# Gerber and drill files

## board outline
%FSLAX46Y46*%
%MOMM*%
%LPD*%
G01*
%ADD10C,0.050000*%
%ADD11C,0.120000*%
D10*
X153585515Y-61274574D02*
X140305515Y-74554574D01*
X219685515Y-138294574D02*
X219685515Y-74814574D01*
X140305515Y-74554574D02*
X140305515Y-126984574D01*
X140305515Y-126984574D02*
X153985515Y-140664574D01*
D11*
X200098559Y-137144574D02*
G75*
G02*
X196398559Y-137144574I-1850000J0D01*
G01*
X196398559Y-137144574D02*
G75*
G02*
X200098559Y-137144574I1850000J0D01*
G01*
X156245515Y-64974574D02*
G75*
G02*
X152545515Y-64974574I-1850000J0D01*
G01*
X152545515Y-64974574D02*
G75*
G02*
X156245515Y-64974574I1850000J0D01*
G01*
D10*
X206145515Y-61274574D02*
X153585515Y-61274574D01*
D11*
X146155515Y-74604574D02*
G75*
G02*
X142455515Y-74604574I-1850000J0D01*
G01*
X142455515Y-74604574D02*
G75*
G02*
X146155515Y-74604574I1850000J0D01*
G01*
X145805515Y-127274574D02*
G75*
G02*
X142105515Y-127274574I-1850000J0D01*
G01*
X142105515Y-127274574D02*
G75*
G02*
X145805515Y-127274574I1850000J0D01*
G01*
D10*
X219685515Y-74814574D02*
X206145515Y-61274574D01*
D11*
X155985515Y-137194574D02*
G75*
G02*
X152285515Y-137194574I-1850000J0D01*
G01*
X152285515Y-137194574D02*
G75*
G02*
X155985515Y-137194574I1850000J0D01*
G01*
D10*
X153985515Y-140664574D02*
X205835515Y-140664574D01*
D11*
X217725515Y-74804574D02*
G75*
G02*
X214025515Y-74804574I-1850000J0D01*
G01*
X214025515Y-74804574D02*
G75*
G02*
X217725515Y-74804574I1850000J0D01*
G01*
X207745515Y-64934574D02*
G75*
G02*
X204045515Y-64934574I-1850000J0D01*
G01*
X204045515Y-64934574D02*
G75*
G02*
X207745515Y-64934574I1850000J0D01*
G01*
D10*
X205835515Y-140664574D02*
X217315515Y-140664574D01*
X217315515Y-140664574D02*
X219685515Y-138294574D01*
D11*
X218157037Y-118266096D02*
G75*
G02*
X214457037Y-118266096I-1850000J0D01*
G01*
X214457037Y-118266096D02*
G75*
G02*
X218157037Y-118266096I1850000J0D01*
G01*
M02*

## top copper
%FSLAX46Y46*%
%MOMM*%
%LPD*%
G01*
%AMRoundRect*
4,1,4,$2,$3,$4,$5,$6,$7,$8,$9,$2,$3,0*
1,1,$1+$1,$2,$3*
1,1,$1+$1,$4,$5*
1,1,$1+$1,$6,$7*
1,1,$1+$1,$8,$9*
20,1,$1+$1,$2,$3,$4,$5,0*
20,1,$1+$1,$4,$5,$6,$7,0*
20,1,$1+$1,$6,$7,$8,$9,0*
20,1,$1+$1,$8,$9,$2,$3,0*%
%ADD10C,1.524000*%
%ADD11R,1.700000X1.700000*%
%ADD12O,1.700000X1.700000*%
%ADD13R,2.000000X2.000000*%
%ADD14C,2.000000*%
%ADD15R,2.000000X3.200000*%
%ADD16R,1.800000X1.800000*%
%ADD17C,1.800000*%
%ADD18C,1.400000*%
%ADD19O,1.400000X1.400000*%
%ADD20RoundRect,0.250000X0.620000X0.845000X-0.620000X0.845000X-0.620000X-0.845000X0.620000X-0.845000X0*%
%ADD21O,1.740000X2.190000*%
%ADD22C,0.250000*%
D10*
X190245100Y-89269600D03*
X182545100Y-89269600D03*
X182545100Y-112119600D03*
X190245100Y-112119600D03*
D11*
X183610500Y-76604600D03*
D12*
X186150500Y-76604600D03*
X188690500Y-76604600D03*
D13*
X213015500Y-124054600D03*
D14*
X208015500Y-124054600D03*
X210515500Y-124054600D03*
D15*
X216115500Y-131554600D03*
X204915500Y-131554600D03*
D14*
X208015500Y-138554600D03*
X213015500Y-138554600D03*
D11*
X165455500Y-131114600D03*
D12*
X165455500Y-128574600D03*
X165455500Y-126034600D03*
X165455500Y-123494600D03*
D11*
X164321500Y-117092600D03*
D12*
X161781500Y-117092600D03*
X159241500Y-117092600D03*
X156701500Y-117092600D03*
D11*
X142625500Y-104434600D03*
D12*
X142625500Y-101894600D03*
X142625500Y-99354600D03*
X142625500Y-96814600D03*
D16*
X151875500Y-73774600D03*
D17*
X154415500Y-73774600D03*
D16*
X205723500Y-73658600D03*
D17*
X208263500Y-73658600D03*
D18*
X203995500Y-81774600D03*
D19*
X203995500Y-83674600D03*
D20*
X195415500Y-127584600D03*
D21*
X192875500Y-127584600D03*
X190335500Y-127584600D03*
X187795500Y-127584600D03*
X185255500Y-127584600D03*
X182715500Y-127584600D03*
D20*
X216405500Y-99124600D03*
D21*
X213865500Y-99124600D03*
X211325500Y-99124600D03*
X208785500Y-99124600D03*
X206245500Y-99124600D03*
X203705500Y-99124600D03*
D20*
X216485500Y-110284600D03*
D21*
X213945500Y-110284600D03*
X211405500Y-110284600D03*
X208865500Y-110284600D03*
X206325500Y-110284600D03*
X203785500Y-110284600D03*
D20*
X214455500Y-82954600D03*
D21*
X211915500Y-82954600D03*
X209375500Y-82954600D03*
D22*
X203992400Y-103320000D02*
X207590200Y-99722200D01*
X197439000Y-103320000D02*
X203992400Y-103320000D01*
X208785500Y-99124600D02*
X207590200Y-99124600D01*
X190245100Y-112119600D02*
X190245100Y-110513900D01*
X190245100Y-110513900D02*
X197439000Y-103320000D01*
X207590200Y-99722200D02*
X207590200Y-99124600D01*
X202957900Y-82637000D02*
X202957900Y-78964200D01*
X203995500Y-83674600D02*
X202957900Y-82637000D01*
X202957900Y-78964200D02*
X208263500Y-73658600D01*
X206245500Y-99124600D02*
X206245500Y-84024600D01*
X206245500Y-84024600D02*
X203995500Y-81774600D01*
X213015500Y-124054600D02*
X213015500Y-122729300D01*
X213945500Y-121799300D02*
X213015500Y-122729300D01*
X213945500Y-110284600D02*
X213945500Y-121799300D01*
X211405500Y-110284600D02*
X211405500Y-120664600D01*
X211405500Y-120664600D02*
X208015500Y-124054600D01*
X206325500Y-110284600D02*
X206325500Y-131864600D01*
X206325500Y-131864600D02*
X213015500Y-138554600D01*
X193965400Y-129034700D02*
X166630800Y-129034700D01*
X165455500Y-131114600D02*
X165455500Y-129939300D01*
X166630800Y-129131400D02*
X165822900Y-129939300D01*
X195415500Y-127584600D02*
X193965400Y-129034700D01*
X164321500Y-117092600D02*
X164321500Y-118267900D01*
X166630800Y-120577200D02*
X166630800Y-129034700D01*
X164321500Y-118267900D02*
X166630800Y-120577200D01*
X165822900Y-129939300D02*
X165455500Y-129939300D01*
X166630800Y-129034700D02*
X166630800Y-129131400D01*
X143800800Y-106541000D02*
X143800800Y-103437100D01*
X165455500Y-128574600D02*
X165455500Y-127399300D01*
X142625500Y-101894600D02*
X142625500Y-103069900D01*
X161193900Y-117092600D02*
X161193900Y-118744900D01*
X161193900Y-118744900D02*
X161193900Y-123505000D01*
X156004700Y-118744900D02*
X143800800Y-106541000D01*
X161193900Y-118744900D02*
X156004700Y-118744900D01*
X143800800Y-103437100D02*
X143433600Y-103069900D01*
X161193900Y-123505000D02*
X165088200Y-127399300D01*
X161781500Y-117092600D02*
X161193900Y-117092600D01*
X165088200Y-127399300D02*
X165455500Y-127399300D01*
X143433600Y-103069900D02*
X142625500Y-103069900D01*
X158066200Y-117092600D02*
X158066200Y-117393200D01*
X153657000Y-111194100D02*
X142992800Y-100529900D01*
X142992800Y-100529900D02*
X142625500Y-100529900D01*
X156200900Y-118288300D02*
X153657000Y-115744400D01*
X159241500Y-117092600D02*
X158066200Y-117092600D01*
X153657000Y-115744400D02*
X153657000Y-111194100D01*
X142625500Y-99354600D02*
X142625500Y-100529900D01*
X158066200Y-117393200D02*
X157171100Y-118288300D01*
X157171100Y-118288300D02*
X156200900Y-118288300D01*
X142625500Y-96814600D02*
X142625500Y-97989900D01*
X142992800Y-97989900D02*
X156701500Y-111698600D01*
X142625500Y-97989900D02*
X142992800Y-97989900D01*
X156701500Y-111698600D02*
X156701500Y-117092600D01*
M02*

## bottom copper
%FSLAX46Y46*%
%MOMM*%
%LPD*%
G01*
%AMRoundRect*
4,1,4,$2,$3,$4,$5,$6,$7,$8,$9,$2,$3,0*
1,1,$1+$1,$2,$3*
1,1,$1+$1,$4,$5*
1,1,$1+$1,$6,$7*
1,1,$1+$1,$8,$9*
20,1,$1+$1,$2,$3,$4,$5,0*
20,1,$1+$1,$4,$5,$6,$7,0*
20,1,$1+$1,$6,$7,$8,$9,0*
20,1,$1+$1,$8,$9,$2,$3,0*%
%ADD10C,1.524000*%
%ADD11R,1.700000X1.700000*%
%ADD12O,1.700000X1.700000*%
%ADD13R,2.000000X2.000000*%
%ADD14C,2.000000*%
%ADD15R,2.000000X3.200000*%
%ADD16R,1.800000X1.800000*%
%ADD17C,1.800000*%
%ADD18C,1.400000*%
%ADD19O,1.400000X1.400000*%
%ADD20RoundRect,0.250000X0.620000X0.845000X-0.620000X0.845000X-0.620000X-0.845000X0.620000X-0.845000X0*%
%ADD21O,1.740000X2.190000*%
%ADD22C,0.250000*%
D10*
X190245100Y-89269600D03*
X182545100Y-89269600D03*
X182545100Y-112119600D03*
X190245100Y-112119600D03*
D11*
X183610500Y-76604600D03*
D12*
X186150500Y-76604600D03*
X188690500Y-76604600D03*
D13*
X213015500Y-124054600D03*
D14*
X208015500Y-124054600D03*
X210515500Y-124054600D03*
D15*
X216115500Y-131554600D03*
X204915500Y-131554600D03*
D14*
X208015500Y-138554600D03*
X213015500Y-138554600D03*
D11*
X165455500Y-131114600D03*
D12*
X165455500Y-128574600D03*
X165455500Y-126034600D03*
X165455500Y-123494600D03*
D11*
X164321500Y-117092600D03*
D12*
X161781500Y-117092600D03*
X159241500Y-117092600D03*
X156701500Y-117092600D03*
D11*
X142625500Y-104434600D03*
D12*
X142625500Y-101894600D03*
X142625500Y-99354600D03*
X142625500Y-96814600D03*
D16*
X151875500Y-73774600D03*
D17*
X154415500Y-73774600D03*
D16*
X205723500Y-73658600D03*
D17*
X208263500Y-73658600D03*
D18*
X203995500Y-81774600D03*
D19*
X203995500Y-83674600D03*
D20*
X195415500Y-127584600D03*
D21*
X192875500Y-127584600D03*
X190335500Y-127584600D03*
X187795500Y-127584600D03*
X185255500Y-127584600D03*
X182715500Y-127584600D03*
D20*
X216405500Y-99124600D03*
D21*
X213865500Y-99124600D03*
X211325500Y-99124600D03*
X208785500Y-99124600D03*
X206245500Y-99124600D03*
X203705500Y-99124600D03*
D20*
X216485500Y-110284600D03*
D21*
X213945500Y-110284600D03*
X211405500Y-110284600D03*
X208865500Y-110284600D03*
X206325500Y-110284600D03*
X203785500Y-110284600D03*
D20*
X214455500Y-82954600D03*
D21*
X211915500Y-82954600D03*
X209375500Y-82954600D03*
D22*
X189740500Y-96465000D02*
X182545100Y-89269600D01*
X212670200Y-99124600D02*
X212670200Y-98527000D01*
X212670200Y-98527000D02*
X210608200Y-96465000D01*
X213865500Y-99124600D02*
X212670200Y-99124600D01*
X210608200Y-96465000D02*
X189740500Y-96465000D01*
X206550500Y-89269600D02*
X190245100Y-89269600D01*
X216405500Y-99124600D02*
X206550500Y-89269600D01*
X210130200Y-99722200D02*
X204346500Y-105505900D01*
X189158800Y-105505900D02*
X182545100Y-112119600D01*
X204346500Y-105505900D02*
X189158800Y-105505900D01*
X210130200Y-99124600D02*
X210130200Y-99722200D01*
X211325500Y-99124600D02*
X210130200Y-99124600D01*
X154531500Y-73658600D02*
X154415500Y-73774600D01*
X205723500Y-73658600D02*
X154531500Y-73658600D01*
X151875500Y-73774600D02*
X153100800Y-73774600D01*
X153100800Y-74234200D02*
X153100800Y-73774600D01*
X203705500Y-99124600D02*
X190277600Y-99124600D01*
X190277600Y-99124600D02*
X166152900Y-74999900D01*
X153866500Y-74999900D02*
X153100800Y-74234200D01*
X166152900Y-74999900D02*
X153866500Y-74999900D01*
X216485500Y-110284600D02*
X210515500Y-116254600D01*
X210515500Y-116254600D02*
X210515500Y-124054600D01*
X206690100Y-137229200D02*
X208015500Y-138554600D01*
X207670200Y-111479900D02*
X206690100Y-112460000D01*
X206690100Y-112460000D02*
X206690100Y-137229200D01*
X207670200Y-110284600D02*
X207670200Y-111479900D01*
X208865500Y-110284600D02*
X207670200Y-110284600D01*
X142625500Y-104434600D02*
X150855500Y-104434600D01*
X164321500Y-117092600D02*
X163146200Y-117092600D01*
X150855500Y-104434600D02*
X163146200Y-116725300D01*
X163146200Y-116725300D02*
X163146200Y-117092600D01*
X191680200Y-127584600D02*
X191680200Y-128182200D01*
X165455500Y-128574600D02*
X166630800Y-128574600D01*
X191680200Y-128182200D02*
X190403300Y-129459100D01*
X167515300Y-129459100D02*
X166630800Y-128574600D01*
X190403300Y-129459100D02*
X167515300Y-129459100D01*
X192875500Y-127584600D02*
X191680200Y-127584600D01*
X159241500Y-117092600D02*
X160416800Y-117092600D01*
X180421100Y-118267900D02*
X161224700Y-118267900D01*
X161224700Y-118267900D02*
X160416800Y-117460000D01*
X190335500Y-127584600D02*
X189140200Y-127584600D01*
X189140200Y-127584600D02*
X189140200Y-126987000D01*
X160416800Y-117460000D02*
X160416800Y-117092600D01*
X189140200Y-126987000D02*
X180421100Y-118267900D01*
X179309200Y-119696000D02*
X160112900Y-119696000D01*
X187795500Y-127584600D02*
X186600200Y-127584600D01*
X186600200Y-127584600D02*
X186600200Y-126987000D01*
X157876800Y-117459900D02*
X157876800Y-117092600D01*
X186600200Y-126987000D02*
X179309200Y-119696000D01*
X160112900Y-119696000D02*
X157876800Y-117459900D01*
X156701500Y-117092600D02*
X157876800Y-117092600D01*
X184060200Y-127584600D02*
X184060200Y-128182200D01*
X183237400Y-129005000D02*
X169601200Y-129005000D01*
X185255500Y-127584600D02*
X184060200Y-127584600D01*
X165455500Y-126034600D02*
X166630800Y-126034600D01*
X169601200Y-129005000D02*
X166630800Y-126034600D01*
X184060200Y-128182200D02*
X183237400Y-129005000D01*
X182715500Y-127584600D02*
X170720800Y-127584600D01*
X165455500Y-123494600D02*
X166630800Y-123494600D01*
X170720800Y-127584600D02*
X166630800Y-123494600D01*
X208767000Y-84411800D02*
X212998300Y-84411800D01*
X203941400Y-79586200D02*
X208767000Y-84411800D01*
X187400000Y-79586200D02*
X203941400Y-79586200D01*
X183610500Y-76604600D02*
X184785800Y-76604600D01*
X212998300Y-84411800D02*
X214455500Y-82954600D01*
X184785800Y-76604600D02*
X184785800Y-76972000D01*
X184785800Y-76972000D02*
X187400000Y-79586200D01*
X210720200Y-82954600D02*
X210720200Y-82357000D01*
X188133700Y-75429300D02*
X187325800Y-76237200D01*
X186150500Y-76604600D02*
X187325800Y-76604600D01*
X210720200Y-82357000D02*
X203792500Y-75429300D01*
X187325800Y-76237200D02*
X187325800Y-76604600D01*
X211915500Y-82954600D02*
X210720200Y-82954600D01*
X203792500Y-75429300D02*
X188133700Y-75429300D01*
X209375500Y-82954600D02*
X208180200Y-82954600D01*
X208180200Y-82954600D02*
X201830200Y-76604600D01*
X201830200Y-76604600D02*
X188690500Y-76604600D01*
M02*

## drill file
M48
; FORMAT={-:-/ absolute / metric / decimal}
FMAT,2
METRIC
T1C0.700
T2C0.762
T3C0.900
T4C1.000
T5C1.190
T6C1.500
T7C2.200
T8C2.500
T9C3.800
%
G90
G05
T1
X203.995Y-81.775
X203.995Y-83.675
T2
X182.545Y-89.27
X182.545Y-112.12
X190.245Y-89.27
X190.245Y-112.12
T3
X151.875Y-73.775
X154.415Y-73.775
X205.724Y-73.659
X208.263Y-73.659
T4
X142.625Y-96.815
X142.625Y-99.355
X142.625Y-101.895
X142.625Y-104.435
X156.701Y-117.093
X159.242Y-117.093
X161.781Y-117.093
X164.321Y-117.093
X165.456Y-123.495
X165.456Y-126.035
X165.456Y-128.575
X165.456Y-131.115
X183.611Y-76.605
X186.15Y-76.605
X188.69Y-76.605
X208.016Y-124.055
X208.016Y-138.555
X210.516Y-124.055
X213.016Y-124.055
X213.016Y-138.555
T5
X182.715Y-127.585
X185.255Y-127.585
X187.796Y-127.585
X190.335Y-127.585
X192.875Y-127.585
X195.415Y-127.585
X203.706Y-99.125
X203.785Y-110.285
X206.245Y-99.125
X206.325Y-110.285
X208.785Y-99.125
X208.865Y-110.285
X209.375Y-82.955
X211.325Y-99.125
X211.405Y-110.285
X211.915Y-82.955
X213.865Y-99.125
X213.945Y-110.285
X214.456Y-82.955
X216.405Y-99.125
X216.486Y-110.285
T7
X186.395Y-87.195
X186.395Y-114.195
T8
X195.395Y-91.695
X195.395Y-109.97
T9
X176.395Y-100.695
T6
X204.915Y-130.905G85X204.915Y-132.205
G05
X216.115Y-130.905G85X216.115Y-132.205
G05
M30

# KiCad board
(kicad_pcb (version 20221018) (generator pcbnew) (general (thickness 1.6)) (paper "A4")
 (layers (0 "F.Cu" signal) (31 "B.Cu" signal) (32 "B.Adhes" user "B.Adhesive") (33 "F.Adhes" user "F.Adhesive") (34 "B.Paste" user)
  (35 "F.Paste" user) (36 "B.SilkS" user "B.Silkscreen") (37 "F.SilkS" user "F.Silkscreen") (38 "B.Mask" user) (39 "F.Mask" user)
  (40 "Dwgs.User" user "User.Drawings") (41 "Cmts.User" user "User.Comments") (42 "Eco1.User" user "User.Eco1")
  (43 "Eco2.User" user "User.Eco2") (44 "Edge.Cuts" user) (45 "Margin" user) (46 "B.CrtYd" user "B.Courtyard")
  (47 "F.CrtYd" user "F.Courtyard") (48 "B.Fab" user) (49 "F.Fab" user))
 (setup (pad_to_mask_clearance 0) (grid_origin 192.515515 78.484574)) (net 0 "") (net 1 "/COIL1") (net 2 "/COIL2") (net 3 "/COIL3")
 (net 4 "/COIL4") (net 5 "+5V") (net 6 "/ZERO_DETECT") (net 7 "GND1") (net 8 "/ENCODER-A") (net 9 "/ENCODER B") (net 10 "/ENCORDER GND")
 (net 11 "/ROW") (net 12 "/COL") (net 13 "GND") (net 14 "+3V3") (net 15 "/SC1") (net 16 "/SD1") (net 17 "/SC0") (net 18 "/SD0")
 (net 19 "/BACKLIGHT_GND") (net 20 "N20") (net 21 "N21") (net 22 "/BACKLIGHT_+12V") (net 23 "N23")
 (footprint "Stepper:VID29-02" (layer "F.Cu") (at 186.3951 100.8596 -90)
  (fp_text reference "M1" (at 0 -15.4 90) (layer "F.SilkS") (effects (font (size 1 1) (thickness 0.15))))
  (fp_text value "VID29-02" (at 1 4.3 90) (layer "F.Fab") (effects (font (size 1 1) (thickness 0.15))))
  (pad "" np_thru_hole circle (at -13.665 0 270) (size 2.2 2.2) (drill 2.2) (layers "*.Cu" "*.Mask"))
  (pad "" np_thru_hole circle (at -9.165 -9 270) (size 2.5 2.5) (drill 2.5) (layers "*.Cu" "*.Mask"))
  (pad "" np_thru_hole circle (at -0.165 10 270) (size 3.8 3.8) (drill 3.8) (layers "*.Cu" "*.Mask"))
  (pad "" np_thru_hole circle (at 9.11 -9 270) (size 2.5 2.5) (drill 2.5) (layers "*.Cu" "*.Mask"))
  (pad "" np_thru_hole circle (at 13.335 0 270) (size 2.2 2.2) (drill 2.2) (layers "*.Cu" "*.Mask"))
  (pad "1" thru_hole circle (at -11.59 -3.85 270) (size 1.524 1.524) (drill 0.762) (layers "*.Cu" "*.Mask") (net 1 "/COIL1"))
  (pad "2" thru_hole circle (at -11.59 3.85 270) (size 1.524 1.524) (drill 0.762) (layers "*.Cu" "*.Mask") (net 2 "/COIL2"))
  (pad "3" thru_hole circle (at 11.26 3.85 270) (size 1.524 1.524) (drill 0.762) (layers "*.Cu" "*.Mask") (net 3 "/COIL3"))
  (pad "4" thru_hole circle (at 11.26 -3.85 270) (size 1.524 1.524) (drill 0.762) (layers "*.Cu" "*.Mask") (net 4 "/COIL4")))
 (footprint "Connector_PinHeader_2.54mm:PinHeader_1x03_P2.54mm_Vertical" (layer "F.Cu") (at 183.6105 76.6046 90)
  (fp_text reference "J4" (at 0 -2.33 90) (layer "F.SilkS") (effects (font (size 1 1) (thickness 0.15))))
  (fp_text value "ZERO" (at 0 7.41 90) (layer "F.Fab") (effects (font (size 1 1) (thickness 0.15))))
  (pad "1" thru_hole rect (at 0 0 90) (size 1.7 1.7) (drill 1) (layers "*.Cu" "*.Mask") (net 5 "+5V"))
  (pad "2" thru_hole oval (at 0 2.54 90) (size 1.7 1.7) (drill 1) (layers "*.Cu" "*.Mask") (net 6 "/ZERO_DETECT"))
  (pad "3" thru_hole oval (at 0 5.08 90) (size 1.7 1.7) (drill 1) (layers "*.Cu" "*.Mask") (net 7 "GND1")))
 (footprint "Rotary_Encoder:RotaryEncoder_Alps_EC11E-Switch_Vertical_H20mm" (layer "F.Cu") (at 213.0155 124.0546 -90)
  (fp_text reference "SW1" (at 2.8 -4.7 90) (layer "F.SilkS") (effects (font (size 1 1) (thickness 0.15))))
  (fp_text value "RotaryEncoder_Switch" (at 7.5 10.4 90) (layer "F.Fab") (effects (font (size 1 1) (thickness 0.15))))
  (pad "A" thru_hole rect (at 0 0 270) (size 2 2) (drill 1) (layers "*.Cu" "*.Mask") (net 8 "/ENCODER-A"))
  (pad "B" thru_hole circle (at 0 5 270) (size 2 2) (drill 1) (layers "*.Cu" "*.Mask") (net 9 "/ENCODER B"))
  (pad "C" thru_hole circle (at 0 2.5 270) (size 2 2) (drill 1) (layers "*.Cu" "*.Mask") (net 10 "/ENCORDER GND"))
  (pad "MP" thru_hole rect (at 7.5 -3.1 270) (size 3.2 2) (drill oval 2.8 1.5) (layers "*.Cu" "*.Mask"))
  (pad "MP" thru_hole rect (at 7.5 8.1 270) (size 3.2 2) (drill oval 2.8 1.5) (layers "*.Cu" "*.Mask"))
  (pad "S1" thru_hole circle (at 14.5 5 270) (size 2 2) (drill 1) (layers "*.Cu" "*.Mask") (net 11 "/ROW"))
  (pad "S2" thru_hole circle (at 14.5 0 270) (size 2 2) (drill 1) (layers "*.Cu" "*.Mask") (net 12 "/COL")))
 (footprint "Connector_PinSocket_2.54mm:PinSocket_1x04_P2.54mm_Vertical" (layer "F.Cu") (at 165.4555 131.1146 180)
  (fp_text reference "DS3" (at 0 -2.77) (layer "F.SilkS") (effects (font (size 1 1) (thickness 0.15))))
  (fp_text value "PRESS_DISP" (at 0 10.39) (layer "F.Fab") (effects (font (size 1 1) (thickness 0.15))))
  (pad "1" thru_hole rect (at 0 0 180) (size 1.7 1.7) (drill 1) (layers "*.Cu" "*.Mask") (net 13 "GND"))
  (pad "2" thru_hole oval (at 0 2.54 180) (size 1.7 1.7) (drill 1) (layers "*.Cu" "*.Mask") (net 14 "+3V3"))
  (pad "3" thru_hole oval (at 0 5.08 180) (size 1.7 1.7) (drill 1) (layers "*.Cu" "*.Mask") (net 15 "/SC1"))
  (pad "4" thru_hole oval (at 0 7.62 180) (size 1.7 1.7) (drill 1) (layers "*.Cu" "*.Mask") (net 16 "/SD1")))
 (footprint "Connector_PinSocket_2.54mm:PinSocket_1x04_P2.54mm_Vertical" (layer "F.Cu") (at 164.3215 117.0926 -90)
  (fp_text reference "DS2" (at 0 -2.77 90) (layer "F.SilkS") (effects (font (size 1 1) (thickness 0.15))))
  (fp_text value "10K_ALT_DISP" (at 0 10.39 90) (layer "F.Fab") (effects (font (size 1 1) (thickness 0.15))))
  (pad "1" thru_hole rect (at 0 0 270) (size 1.7 1.7) (drill 1) (layers "*.Cu" "*.Mask") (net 13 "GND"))
  (pad "2" thru_hole oval (at 0 2.54 270) (size 1.7 1.7) (drill 1) (layers "*.Cu" "*.Mask") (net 14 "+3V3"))
  (pad "3" thru_hole oval (at 0 5.08 270) (size 1.7 1.7) (drill 1) (layers "*.Cu" "*.Mask") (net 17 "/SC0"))
  (pad "4" thru_hole oval (at 0 7.62 270) (size 1.7 1.7) (drill 1) (layers "*.Cu" "*.Mask") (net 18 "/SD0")))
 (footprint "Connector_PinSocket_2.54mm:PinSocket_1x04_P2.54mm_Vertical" (layer "F.Cu") (at 142.6255 104.4346 180)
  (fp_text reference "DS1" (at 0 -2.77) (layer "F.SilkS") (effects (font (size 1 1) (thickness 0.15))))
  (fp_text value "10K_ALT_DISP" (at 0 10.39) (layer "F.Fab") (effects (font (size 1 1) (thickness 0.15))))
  (pad "1" thru_hole rect (at 0 0 180) (size 1.7 1.7) (drill 1) (layers "*.Cu" "*.Mask") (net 13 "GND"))
  (pad "2" thru_hole oval (at 0 2.54 180) (size 1.7 1.7) (drill 1) (layers "*.Cu" "*.Mask") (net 14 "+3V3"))
  (pad "3" thru_hole oval (at 0 5.08 180) (size 1.7 1.7) (drill 1) (layers "*.Cu" "*.Mask") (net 17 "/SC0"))
  (pad "4" thru_hole oval (at 0 7.62 180) (size 1.7 1.7) (drill 1) (layers "*.Cu" "*.Mask") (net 18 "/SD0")))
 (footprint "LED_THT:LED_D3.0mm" (layer "F.Cu") (at 151.8755 73.7746)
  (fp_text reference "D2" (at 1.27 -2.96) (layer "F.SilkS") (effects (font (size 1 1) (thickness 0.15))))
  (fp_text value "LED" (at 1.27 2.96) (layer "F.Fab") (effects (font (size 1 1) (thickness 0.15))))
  (pad "1" thru_hole rect (at 0 0) (size 1.8 1.8) (drill 0.9) (layers "*.Cu" "*.Mask") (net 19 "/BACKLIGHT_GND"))
  (pad "2" thru_hole circle (at 2.54 0) (size 1.8 1.8) (drill 0.9) (layers "*.Cu" "*.Mask") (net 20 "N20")))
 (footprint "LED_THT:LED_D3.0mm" (layer "F.Cu") (at 205.7235 73.6586)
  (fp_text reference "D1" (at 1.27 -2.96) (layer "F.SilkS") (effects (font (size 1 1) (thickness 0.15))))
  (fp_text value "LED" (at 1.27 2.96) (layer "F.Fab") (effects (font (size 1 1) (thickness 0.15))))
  (pad "1" thru_hole rect (at 0 0) (size 1.8 1.8) (drill 0.9) (layers "*.Cu" "*.Mask") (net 20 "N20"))
  (pad "2" thru_hole circle (at 2.54 0) (size 1.8 1.8) (drill 0.9) (layers "*.Cu" "*.Mask") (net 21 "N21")))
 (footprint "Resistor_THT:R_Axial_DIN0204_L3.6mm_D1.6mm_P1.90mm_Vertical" (layer "B.Cu") (at 203.9955 81.7746 -90)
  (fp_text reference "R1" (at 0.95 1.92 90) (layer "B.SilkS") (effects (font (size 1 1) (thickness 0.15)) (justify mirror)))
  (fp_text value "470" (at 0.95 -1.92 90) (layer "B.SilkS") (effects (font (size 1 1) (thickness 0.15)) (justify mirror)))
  (pad "1" thru_hole circle (at 0 0 270) (size 1.4 1.4) (drill 0.7) (layers "*.Cu" "*.Mask") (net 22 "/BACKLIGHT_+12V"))
  (pad "2" thru_hole oval (at 1.9 0 270) (size 1.4 1.4) (drill 0.7) (layers "*.Cu" "*.Mask") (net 21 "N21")))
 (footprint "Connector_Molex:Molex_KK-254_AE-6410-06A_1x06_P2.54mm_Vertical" (layer "B.Cu") (at 195.4155 127.5846 180)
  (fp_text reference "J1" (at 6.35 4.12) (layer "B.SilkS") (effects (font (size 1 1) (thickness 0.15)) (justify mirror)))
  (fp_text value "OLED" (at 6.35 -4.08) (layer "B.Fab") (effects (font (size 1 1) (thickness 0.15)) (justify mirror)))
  (pad "1" thru_hole roundrect (at 0 0 180) (size 1.74 2.19) (drill 1.19) (layers "*.Cu" "*.Mask") (roundrect_rratio 0.1436781609)
   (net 13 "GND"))
  (pad "2" thru_hole oval (at 2.54 0 180) (size 1.74 2.19) (drill 1.19) (layers "*.Cu" "*.Mask") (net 14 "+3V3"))
  (pad "3" thru_hole oval (at 5.08 0 180) (size 1.74 2.19) (drill 1.19) (layers "*.Cu" "*.Mask") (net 17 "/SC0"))
  (pad "4" thru_hole oval (at 7.62 0 180) (size 1.74 2.19) (drill 1.19) (layers "*.Cu" "*.Mask") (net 18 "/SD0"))
  (pad "5" thru_hole oval (at 10.16 0 180) (size 1.74 2.19) (drill 1.19) (layers "*.Cu" "*.Mask") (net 15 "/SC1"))
  (pad "6" thru_hole oval (at 12.7 0 180) (size 1.74 2.19) (drill 1.19) (layers "*.Cu" "*.Mask") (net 16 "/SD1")))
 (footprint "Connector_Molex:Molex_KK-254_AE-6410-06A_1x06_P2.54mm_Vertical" (layer "B.Cu") (at 216.4055 99.1246 180)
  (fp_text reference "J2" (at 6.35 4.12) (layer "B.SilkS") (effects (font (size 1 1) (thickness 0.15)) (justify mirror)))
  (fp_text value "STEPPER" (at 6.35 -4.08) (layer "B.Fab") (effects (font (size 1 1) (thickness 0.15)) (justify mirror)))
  (pad "1" thru_hole roundrect (at 0 0 180) (size 1.74 2.19) (drill 1.19) (layers "*.Cu" "*.Mask") (roundrect_rratio 0.1436781609)
   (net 1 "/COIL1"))
  (pad "2" thru_hole oval (at 2.54 0 180) (size 1.74 2.19) (drill 1.19) (layers "*.Cu" "*.Mask") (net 2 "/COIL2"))
  (pad "3" thru_hole oval (at 5.08 0 180) (size 1.74 2.19) (drill 1.19) (layers "*.Cu" "*.Mask") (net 3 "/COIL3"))
  (pad "4" thru_hole oval (at 7.62 0 180) (size 1.74 2.19) (drill 1.19) (layers "*.Cu" "*.Mask") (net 4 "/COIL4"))
  (pad "5" thru_hole oval (at 10.16 0 180) (size 1.74 2.19) (drill 1.19) (layers "*.Cu" "*.Mask") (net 22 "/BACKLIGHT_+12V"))
  (pad "6" thru_hole oval (at 12.7 0 180) (size 1.74 2.19) (drill 1.19) (layers "*.Cu" "*.Mask") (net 19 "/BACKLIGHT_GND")))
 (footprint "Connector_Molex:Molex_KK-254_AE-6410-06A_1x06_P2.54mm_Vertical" (layer "B.Cu") (at 216.4855 110.2846 180)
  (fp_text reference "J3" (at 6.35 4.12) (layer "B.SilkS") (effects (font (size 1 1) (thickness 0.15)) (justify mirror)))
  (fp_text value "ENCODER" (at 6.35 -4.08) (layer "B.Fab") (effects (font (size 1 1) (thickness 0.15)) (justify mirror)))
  (pad "1" thru_hole roundrect (at 0 0 180) (size 1.74 2.19) (drill 1.19) (layers "*.Cu" "*.Mask") (roundrect_rratio 0.1436781609)
   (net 10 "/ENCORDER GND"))
  (pad "2" thru_hole oval (at 2.54 0 180) (size 1.74 2.19) (drill 1.19) (layers "*.Cu" "*.Mask") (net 8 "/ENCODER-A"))
  (pad "3" thru_hole oval (at 5.08 0 180) (size 1.74 2.19) (drill 1.19) (layers "*.Cu" "*.Mask") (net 9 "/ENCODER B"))
  (pad "4" thru_hole oval (at 7.62 0 180) (size 1.74 2.19) (drill 1.19) (layers "*.Cu" "*.Mask") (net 11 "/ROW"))
  (pad "5" thru_hole oval (at 10.16 0 180) (size 1.74 2.19) (drill 1.19) (layers "*.Cu" "*.Mask") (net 12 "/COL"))
  (pad "6" thru_hole oval (at 12.7 0 180) (size 1.74 2.19) (drill 1.19) (layers "*.Cu" "*.Mask") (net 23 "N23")))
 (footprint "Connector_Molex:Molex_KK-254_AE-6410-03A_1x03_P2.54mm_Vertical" (layer "B.Cu") (at 214.4555 82.9546 180)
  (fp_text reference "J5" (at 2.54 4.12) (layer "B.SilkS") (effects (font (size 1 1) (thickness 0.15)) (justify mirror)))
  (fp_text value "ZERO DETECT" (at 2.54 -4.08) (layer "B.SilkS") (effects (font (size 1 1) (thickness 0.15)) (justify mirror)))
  (pad "1" thru_hole roundrect (at 0 0 180) (size 1.74 2.19) (drill 1.19) (layers "*.Cu" "*.Mask") (roundrect_rratio 0.1436781609)
   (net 5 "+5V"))
  (pad "2" thru_hole oval (at 2.54 0 180) (size 1.74 2.19) (drill 1.19) (layers "*.Cu" "*.Mask") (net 6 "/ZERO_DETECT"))
  (pad "3" thru_hole oval (at 5.08 0 180) (size 1.74 2.19) (drill 1.19) (layers "*.Cu" "*.Mask") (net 7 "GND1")))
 (gr_line (start 153.585515 61.274574) (end 140.305515 74.554574) (stroke (width 0.05) (type solid)) (layer "Edge.Cuts"))
 (gr_line (start 219.685515 138.294574) (end 219.685515 74.814574) (stroke (width 0.05) (type solid)) (layer "Edge.Cuts"))
 (gr_line (start 140.305515 74.554574) (end 140.305515 126.984574) (stroke (width 0.05) (type solid)) (layer "Edge.Cuts"))
 (gr_line (start 140.305515 126.984574) (end 153.985515 140.664574) (stroke (width 0.05) (type solid)) (layer "Edge.Cuts"))
 (gr_circle (center 198.248559 137.144574) (end 200.098559 137.144574) (stroke (width 0.12) (type solid)) (fill none) (layer "Edge.Cuts"))
 (gr_circle (center 154.395515 64.974574) (end 156.245515 64.974574) (stroke (width 0.12) (type solid)) (fill none) (layer "Edge.Cuts"))
 (gr_line (start 206.145515 61.274574) (end 153.585515 61.274574) (stroke (width 0.05) (type solid)) (layer "Edge.Cuts"))
 (gr_circle (center 144.305515 74.604574) (end 146.155515 74.604574) (stroke (width 0.12) (type solid)) (fill none) (layer "Edge.Cuts"))
 (gr_circle (center 143.955515 127.274574) (end 145.805515 127.274574) (stroke (width 0.12) (type solid)) (fill none) (layer "Edge.Cuts"))
 (gr_line (start 219.685515 74.814574) (end 206.145515 61.274574) (stroke (width 0.05) (type solid)) (layer "Edge.Cuts"))
 (gr_circle (center 154.135515 137.194574) (end 155.985515 137.194574) (stroke (width 0.12) (type solid)) (fill none) (layer "Edge.Cuts"))
 (gr_line (start 153.985515 140.664574) (end 205.835515 140.664574) (stroke (width 0.05) (type solid)) (layer "Edge.Cuts"))
 (gr_circle (center 215.875515 74.804574) (end 217.725515 74.804574) (stroke (width 0.12) (type solid)) (fill none) (layer "Edge.Cuts"))
 (gr_circle (center 205.895515 64.934574) (end 207.745515 64.934574) (stroke (width 0.12) (type solid)) (fill none) (layer "Edge.Cuts"))
 (gr_line (start 205.835515 140.664574) (end 217.315515 140.664574) (stroke (width 0.05) (type solid)) (layer "Edge.Cuts"))
 (gr_line (start 217.315515 140.664574) (end 219.685515 138.294574) (stroke (width 0.05) (type solid)) (layer "Edge.Cuts"))
 (gr_circle (center 216.307037 118.266096) (end 218.157037 118.266096) (stroke (width 0.12) (type solid)) (fill none) (layer "Edge.Cuts"))
 (segment (start 189.7405 96.465) (end 182.5451 89.2696) (width 0.25) (layer "B.Cu") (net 2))
 (segment (start 212.6702 99.1246) (end 212.6702 98.527) (width 0.25) (layer "B.Cu") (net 2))
 (segment (start 212.6702 98.527) (end 210.6082 96.465) (width 0.25) (layer "B.Cu") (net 2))
 (segment (start 213.8655 99.1246) (end 212.6702 99.1246) (width 0.25) (layer "B.Cu") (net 2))
 (segment (start 210.6082 96.465) (end 189.7405 96.465) (width 0.25) (layer "B.Cu") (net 2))
 (segment (start 206.5505 89.2696) (end 190.2451 89.2696) (width 0.25) (layer "B.Cu") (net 1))
 (segment (start 216.4055 99.1246) (end 206.5505 89.2696) (width 0.25) (layer "B.Cu") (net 1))
 (segment (start 203.9924 103.32) (end 207.5902 99.7222) (width 0.25) (layer "F.Cu") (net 4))
 (segment (start 197.439 103.32) (end 203.9924 103.32) (width 0.25) (layer "F.Cu") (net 4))
 (segment (start 208.7855 99.1246) (end 207.5902 99.1246) (width 0.25) (layer "F.Cu") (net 4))
 (segment (start 190.2451 112.1196) (end 190.2451 110.5139) (width 0.25) (layer "F.Cu") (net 4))
 (segment (start 190.2451 110.5139) (end 197.439 103.32) (width 0.25) (layer "F.Cu") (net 4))
 (segment (start 207.5902 99.7222) (end 207.5902 99.1246) (width 0.25) (layer "F.Cu") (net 4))
 (segment (start 210.1302 99.7222) (end 204.3465 105.5059) (width 0.25) (layer "B.Cu") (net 3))
 (segment (start 189.1588 105.5059) (end 182.5451 112.1196) (width 0.25) (layer "B.Cu") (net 3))
 (segment (start 204.3465 105.5059) (end 189.1588 105.5059) (width 0.25) (layer "B.Cu") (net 3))
 (segment (start 210.1302 99.1246) (end 210.1302 99.7222) (width 0.25) (layer "B.Cu") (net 3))
 (segment (start 211.3255 99.1246) (end 210.1302 99.1246) (width 0.25) (layer "B.Cu") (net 3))
 (segment (start 154.5315 73.6586) (end 154.4155 73.7746) (width 0.25) (layer "B.Cu") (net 20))
 (segment (start 205.7235 73.6586) (end 154.5315 73.6586) (width 0.25) (layer "B.Cu") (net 20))
 (segment (start 202.9579 82.637) (end 202.9579 78.9642) (width 0.25) (layer "F.Cu") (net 21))
 (segment (start 203.9955 83.6746) (end 202.9579 82.637) (width 0.25) (layer "F.Cu") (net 21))
 (segment (start 202.9579 78.9642) (end 208.2635 73.6586) (width 0.25) (layer "F.Cu") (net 21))
 (segment (start 151.8755 73.7746) (end 153.1008 73.7746) (width 0.25) (layer "B.Cu") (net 19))
 (segment (start 153.1008 74.2342) (end 153.1008 73.7746) (width 0.25) (layer "B.Cu") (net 19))
 (segment (start 203.7055 99.1246) (end 190.2776 99.1246) (width 0.25) (layer "B.Cu") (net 19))
 (segment (start 190.2776 99.1246) (end 166.1529 74.9999) (width 0.25) (layer "B.Cu") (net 19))
 (segment (start 153.8665 74.9999) (end 153.1008 74.2342) (width 0.25) (layer "B.Cu") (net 19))
 (segment (start 166.1529 74.9999) (end 153.8665 74.9999) (width 0.25) (layer "B.Cu") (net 19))
 (segment (start 206.2455 99.1246) (end 206.2455 84.0246) (width 0.25) (layer "F.Cu") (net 22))
 (segment (start 206.2455 84.0246) (end 203.9955 81.7746) (width 0.25) (layer "F.Cu") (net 22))
 (segment (start 216.4855 110.2846) (end 210.5155 116.2546) (width 0.25) (layer "B.Cu") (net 10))
 (segment (start 210.5155 116.2546) (end 210.5155 124.0546) (width 0.25) (layer "B.Cu") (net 10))
 (segment (start 213.0155 124.0546) (end 213.0155 122.7293) (width 0.25) (layer "F.Cu") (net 8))
 (segment (start 213.9455 121.7993) (end 213.0155 122.7293) (width 0.25) (layer "F.Cu") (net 8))
 (segment (start 213.9455 110.2846) (end 213.9455 121.7993) (width 0.25) (layer "F.Cu") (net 8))
 (segment (start 211.4055 110.2846) (end 211.4055 120.6646) (width 0.25) (layer "F.Cu") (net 9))
 (segment (start 211.4055 120.6646) (end 208.0155 124.0546) (width 0.25) (layer "F.Cu") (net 9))
 (segment (start 206.6901 137.2292) (end 208.0155 138.5546) (width 0.25) (layer "B.Cu") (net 11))
 (segment (start 207.6702 111.4799) (end 206.6901 112.46) (width 0.25) (layer "B.Cu") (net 11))
 (segment (start 206.6901 112.46) (end 206.6901 137.2292) (width 0.25) (layer "B.Cu") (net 11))
 (segment (start 207.6702 110.2846) (end 207.6702 111.4799) (width 0.25) (layer "B.Cu") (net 11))
 (segment (start 208.8655 110.2846) (end 207.6702 110.2846) (width 0.25) (layer "B.Cu") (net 11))
 (segment (start 206.3255 110.2846) (end 206.3255 131.8646) (width 0.25) (layer "F.Cu") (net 12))
 (segment (start 206.3255 131.8646) (end 213.0155 138.5546) (width 0.25) (layer "F.Cu") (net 12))
 (segment (start 193.9654 129.0347) (end 166.6308 129.0347) (width 0.25) (layer "F.Cu") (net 13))
 (segment (start 165.4555 131.1146) (end 165.4555 129.9393) (width 0.25) (layer "F.Cu") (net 13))
 (segment (start 166.6308 129.1314) (end 165.8229 129.9393) (width 0.25) (layer "F.Cu") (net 13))
 (segment (start 195.4155 127.5846) (end 193.9654 129.0347) (width 0.25) (layer "F.Cu") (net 13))
 (segment (start 164.3215 117.0926) (end 164.3215 118.2679) (width 0.25) (layer "F.Cu") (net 13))
 (segment (start 166.6308 120.5772) (end 166.6308 129.0347) (width 0.25) (layer "F.Cu") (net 13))
 (segment (start 164.3215 118.2679) (end 166.6308 120.5772) (width 0.25) (layer "F.Cu") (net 13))
 (segment (start 165.8229 129.9393) (end 165.4555 129.9393) (width 0.25) (layer "F.Cu") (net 13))
 (segment (start 166.6308 129.0347) (end 166.6308 129.1314) (width 0.25) (layer "F.Cu") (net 13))
 (segment (start 142.6255 104.4346) (end 150.8555 104.4346) (width 0.25) (layer "B.Cu") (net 13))
 (segment (start 164.3215 117.0926) (end 163.1462 117.0926) (width 0.25) (layer "B.Cu") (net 13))
 (segment (start 150.8555 104.4346) (end 163.1462 116.7253) (width 0.25) (layer "B.Cu") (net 13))
 (segment (start 163.1462 116.7253) (end 163.1462 117.0926) (width 0.25) (layer "B.Cu") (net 13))
 (segment (start 143.8008 106.541) (end 143.8008 103.4371) (width 0.25) (layer "F.Cu") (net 14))
 (segment (start 165.4555 128.5746) (end 165.4555 127.3993) (width 0.25) (layer "F.Cu") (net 14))
 (segment (start 142.6255 101.8946) (end 142.6255 103.0699) (width 0.25) (layer "F.Cu") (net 14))
 (segment (start 161.1939 117.0926) (end 161.1939 118.7449) (width 0.25) (layer "F.Cu") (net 14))
 (segment (start 161.1939 118.7449) (end 161.1939 123.505) (width 0.25) (layer "F.Cu") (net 14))
 (segment (start 156.0047 118.7449) (end 143.8008 106.541) (width 0.25) (layer "F.Cu") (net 14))
 (segment (start 161.1939 118.7449) (end 156.0047 118.7449) (width 0.25) (layer "F.Cu") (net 14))
 (segment (start 143.8008 103.4371) (end 143.4336 103.0699) (width 0.25) (layer "F.Cu") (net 14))
 (segment (start 161.1939 123.505) (end 165.0882 127.3993) (width 0.25) (layer "F.Cu") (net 14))
 (segment (start 161.7815 117.0926) (end 161.1939 117.0926) (width 0.25) (layer "F.Cu") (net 14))
 (segment (start 165.0882 127.3993) (end 165.4555 127.3993) (width 0.25) (layer "F.Cu") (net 14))
 (segment (start 143.4336 103.0699) (end 142.6255 103.0699) (width 0.25) (layer "F.Cu") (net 14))
 (segment (start 191.6802 127.5846) (end 191.6802 128.1822) (width 0.25) (layer "B.Cu") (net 14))
 (segment (start 165.4555 128.5746) (end 166.6308 128.5746) (width 0.25) (layer "B.Cu") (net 14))
 (segment (start 191.6802 128.1822) (end 190.4033 129.4591) (width 0.25) (layer "B.Cu") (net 14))
 (segment (start 167.5153 129.4591) (end 166.6308 128.5746) (width 0.25) (layer "B.Cu") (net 14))
 (segment (start 190.4033 129.4591) (end 167.5153 129.4591) (width 0.25) (layer "B.Cu") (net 14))
 (segment (start 192.8755 127.5846) (end 191.6802 127.5846) (width 0.25) (layer "B.Cu") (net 14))
 (segment (start 158.0662 117.0926) (end 158.0662 117.3932) (width 0.25) (layer "F.Cu") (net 17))
 (segment (start 153.657 111.1941) (end 142.9928 100.5299) (width 0.25) (layer "F.Cu") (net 17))
 (segment (start 142.9928 100.5299) (end 142.6255 100.5299) (width 0.25) (layer "F.Cu") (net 17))
 (segment (start 156.2009 118.2883) (end 153.657 115.7444) (width 0.25) (layer "F.Cu") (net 17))
 (segment (start 159.2415 117.0926) (end 158.0662 117.0926) (width 0.25) (layer "F.Cu") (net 17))
 (segment (start 153.657 115.7444) (end 153.657 111.1941) (width 0.25) (layer "F.Cu") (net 17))
 (segment (start 142.6255 99.3546) (end 142.6255 100.5299) (width 0.25) (layer "F.Cu") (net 17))
 (segment (start 158.0662 117.3932) (end 157.1711 118.2883) (width 0.25) (layer "F.Cu") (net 17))
 (segment (start 157.1711 118.2883) (end 156.2009 118.2883) (width 0.25) (layer "F.Cu") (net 17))
 (segment (start 159.2415 117.0926) (end 160.4168 117.0926) (width 0.25) (layer "B.Cu") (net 17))
 (segment (start 180.4211 118.2679) (end 161.2247 118.2679) (width 0.25) (layer "B.Cu") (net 17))
 (segment (start 161.2247 118.2679) (end 160.4168 117.46) (width 0.25) (layer "B.Cu") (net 17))
 (segment (start 190.3355 127.5846) (end 189.1402 127.5846) (width 0.25) (layer "B.Cu") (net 17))
 (segment (start 189.1402 127.5846) (end 189.1402 126.987) (width 0.25) (layer "B.Cu") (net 17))
 (segment (start 160.4168 117.46) (end 160.4168 117.0926) (width 0.25) (layer "B.Cu") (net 17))
 (segment (start 189.1402 126.987) (end 180.4211 118.2679) (width 0.25) (layer "B.Cu") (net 17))
 (segment (start 142.6255 96.8146) (end 142.6255 97.9899) (width 0.25) (layer "F.Cu") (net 18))
 (segment (start 142.9928 97.9899) (end 156.7015 111.6986) (width 0.25) (layer "F.Cu") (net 18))
 (segment (start 142.6255 97.9899) (end 142.9928 97.9899) (width 0.25) (layer "F.Cu") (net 18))
 (segment (start 156.7015 111.6986) (end 156.7015 117.0926) (width 0.25) (layer "F.Cu") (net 18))
 (segment (start 179.3092 119.696) (end 160.1129 119.696) (width 0.25) (layer "B.Cu") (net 18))
 (segment (start 187.7955 127.5846) (end 186.6002 127.5846) (width 0.25) (layer "B.Cu") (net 18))
 (segment (start 186.6002 127.5846) (end 186.6002 126.987) (width 0.25) (layer "B.Cu") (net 18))
 (segment (start 157.8768 117.4599) (end 157.8768 117.0926) (width 0.25) (layer "B.Cu") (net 18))
 (segment (start 186.6002 126.987) (end 179.3092 119.696) (width 0.25) (layer "B.Cu") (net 18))
 (segment (start 160.1129 119.696) (end 157.8768 117.4599) (width 0.25) (layer "B.Cu") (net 18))
 (segment (start 156.7015 117.0926) (end 157.8768 117.0926) (width 0.25) (layer "B.Cu") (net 18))
 (segment (start 184.0602 127.5846) (end 184.0602 128.1822) (width 0.25) (layer "B.Cu") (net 15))
 (segment (start 183.2374 129.005) (end 169.6012 129.005) (width 0.25) (layer "B.Cu") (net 15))
 (segment (start 185.2555 127.5846) (end 184.0602 127.5846) (width 0.25) (layer "B.Cu") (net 15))
 (segment (start 165.4555 126.0346) (end 166.6308 126.0346) (width 0.25) (layer "B.Cu") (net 15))
 (segment (start 169.6012 129.005) (end 166.6308 126.0346) (width 0.25) (layer "B.Cu") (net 15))
 (segment (start 184.0602 128.1822) (end 183.2374 129.005) (width 0.25) (layer "B.Cu") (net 15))
 (segment (start 182.7155 127.5846) (end 170.7208 127.5846) (width 0.25) (layer "B.Cu") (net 16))
 (segment (start 165.4555 123.4946) (end 166.6308 123.4946) (width 0.25) (layer "B.Cu") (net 16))
 (segment (start 170.7208 127.5846) (end 166.6308 123.4946) (width 0.25) (layer "B.Cu") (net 16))
 (segment (start 208.767 84.4118) (end 212.9983 84.4118) (width 0.25) (layer "B.Cu") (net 5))
 (segment (start 203.9414 79.5862) (end 208.767 84.4118) (width 0.25) (layer "B.Cu") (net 5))
 (segment (start 187.4 79.5862) (end 203.9414 79.5862) (width 0.25) (layer "B.Cu") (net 5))
 (segment (start 183.6105 76.6046) (end 184.7858 76.6046) (width 0.25) (layer "B.Cu") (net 5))
 (segment (start 212.9983 84.4118) (end 214.4555 82.9546) (width 0.25) (layer "B.Cu") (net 5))
 (segment (start 184.7858 76.6046) (end 184.7858 76.972) (width 0.25) (layer "B.Cu") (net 5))
 (segment (start 184.7858 76.972) (end 187.4 79.5862) (width 0.25) (layer "B.Cu") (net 5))
 (segment (start 210.7202 82.9546) (end 210.7202 82.357) (width 0.25) (layer "B.Cu") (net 6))
 (segment (start 188.1337 75.4293) (end 187.3258 76.2372) (width 0.25) (layer "B.Cu") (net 6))
 (segment (start 186.1505 76.6046) (end 187.3258 76.6046) (width 0.25) (layer "B.Cu") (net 6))
 (segment (start 210.7202 82.357) (end 203.7925 75.4293) (width 0.25) (layer "B.Cu") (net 6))
 (segment (start 187.3258 76.2372) (end 187.3258 76.6046) (width 0.25) (layer "B.Cu") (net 6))
 (segment (start 211.9155 82.9546) (end 210.7202 82.9546) (width 0.25) (layer "B.Cu") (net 6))
 (segment (start 203.7925 75.4293) (end 188.1337 75.4293) (width 0.25) (layer "B.Cu") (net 6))
 (segment (start 209.3755 82.9546) (end 208.1802 82.9546) (width 0.25) (layer "B.Cu") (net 7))
 (segment (start 208.1802 82.9546) (end 201.8302 76.6046) (width 0.25) (layer "B.Cu") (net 7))
 (segment (start 201.8302 76.6046) (end 188.6905 76.6046) (width 0.25) (layer "B.Cu") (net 7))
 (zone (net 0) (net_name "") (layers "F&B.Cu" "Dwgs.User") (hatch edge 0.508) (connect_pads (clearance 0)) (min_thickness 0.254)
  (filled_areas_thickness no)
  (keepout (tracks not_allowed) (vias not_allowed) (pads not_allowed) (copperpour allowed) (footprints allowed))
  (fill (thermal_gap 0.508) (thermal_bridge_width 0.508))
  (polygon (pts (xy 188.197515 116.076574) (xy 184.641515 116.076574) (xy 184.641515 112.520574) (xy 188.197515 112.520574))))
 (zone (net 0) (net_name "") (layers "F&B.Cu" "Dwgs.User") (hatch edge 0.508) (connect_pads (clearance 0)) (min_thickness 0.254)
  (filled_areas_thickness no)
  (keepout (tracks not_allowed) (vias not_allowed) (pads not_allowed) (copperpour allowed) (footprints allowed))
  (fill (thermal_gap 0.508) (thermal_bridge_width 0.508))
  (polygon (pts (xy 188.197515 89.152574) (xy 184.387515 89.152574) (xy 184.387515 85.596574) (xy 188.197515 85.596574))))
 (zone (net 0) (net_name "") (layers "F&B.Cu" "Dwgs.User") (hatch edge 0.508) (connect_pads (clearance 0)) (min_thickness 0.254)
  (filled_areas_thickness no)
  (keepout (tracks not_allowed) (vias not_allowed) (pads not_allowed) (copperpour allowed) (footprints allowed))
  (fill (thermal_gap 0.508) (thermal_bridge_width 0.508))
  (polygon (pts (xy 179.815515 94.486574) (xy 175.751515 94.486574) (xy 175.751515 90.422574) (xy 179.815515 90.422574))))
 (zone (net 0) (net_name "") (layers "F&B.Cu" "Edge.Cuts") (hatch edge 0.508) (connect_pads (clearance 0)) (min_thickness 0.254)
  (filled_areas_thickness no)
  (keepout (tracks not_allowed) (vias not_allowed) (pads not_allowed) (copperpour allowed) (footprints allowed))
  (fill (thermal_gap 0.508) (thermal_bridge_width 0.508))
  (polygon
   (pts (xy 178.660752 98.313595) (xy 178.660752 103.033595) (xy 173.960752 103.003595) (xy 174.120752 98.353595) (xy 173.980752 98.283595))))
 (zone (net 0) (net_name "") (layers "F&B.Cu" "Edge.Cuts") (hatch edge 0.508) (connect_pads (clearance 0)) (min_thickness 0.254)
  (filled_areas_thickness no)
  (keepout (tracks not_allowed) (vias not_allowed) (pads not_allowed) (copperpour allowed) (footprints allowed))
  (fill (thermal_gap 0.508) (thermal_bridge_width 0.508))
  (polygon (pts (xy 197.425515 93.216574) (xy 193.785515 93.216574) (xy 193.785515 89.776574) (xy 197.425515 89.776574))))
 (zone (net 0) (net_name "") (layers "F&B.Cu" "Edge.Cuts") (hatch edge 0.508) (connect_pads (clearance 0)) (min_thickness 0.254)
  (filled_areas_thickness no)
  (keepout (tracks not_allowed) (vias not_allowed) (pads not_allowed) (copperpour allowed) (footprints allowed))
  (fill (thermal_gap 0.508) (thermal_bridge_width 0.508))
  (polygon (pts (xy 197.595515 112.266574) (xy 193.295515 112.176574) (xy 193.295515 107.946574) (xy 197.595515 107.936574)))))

